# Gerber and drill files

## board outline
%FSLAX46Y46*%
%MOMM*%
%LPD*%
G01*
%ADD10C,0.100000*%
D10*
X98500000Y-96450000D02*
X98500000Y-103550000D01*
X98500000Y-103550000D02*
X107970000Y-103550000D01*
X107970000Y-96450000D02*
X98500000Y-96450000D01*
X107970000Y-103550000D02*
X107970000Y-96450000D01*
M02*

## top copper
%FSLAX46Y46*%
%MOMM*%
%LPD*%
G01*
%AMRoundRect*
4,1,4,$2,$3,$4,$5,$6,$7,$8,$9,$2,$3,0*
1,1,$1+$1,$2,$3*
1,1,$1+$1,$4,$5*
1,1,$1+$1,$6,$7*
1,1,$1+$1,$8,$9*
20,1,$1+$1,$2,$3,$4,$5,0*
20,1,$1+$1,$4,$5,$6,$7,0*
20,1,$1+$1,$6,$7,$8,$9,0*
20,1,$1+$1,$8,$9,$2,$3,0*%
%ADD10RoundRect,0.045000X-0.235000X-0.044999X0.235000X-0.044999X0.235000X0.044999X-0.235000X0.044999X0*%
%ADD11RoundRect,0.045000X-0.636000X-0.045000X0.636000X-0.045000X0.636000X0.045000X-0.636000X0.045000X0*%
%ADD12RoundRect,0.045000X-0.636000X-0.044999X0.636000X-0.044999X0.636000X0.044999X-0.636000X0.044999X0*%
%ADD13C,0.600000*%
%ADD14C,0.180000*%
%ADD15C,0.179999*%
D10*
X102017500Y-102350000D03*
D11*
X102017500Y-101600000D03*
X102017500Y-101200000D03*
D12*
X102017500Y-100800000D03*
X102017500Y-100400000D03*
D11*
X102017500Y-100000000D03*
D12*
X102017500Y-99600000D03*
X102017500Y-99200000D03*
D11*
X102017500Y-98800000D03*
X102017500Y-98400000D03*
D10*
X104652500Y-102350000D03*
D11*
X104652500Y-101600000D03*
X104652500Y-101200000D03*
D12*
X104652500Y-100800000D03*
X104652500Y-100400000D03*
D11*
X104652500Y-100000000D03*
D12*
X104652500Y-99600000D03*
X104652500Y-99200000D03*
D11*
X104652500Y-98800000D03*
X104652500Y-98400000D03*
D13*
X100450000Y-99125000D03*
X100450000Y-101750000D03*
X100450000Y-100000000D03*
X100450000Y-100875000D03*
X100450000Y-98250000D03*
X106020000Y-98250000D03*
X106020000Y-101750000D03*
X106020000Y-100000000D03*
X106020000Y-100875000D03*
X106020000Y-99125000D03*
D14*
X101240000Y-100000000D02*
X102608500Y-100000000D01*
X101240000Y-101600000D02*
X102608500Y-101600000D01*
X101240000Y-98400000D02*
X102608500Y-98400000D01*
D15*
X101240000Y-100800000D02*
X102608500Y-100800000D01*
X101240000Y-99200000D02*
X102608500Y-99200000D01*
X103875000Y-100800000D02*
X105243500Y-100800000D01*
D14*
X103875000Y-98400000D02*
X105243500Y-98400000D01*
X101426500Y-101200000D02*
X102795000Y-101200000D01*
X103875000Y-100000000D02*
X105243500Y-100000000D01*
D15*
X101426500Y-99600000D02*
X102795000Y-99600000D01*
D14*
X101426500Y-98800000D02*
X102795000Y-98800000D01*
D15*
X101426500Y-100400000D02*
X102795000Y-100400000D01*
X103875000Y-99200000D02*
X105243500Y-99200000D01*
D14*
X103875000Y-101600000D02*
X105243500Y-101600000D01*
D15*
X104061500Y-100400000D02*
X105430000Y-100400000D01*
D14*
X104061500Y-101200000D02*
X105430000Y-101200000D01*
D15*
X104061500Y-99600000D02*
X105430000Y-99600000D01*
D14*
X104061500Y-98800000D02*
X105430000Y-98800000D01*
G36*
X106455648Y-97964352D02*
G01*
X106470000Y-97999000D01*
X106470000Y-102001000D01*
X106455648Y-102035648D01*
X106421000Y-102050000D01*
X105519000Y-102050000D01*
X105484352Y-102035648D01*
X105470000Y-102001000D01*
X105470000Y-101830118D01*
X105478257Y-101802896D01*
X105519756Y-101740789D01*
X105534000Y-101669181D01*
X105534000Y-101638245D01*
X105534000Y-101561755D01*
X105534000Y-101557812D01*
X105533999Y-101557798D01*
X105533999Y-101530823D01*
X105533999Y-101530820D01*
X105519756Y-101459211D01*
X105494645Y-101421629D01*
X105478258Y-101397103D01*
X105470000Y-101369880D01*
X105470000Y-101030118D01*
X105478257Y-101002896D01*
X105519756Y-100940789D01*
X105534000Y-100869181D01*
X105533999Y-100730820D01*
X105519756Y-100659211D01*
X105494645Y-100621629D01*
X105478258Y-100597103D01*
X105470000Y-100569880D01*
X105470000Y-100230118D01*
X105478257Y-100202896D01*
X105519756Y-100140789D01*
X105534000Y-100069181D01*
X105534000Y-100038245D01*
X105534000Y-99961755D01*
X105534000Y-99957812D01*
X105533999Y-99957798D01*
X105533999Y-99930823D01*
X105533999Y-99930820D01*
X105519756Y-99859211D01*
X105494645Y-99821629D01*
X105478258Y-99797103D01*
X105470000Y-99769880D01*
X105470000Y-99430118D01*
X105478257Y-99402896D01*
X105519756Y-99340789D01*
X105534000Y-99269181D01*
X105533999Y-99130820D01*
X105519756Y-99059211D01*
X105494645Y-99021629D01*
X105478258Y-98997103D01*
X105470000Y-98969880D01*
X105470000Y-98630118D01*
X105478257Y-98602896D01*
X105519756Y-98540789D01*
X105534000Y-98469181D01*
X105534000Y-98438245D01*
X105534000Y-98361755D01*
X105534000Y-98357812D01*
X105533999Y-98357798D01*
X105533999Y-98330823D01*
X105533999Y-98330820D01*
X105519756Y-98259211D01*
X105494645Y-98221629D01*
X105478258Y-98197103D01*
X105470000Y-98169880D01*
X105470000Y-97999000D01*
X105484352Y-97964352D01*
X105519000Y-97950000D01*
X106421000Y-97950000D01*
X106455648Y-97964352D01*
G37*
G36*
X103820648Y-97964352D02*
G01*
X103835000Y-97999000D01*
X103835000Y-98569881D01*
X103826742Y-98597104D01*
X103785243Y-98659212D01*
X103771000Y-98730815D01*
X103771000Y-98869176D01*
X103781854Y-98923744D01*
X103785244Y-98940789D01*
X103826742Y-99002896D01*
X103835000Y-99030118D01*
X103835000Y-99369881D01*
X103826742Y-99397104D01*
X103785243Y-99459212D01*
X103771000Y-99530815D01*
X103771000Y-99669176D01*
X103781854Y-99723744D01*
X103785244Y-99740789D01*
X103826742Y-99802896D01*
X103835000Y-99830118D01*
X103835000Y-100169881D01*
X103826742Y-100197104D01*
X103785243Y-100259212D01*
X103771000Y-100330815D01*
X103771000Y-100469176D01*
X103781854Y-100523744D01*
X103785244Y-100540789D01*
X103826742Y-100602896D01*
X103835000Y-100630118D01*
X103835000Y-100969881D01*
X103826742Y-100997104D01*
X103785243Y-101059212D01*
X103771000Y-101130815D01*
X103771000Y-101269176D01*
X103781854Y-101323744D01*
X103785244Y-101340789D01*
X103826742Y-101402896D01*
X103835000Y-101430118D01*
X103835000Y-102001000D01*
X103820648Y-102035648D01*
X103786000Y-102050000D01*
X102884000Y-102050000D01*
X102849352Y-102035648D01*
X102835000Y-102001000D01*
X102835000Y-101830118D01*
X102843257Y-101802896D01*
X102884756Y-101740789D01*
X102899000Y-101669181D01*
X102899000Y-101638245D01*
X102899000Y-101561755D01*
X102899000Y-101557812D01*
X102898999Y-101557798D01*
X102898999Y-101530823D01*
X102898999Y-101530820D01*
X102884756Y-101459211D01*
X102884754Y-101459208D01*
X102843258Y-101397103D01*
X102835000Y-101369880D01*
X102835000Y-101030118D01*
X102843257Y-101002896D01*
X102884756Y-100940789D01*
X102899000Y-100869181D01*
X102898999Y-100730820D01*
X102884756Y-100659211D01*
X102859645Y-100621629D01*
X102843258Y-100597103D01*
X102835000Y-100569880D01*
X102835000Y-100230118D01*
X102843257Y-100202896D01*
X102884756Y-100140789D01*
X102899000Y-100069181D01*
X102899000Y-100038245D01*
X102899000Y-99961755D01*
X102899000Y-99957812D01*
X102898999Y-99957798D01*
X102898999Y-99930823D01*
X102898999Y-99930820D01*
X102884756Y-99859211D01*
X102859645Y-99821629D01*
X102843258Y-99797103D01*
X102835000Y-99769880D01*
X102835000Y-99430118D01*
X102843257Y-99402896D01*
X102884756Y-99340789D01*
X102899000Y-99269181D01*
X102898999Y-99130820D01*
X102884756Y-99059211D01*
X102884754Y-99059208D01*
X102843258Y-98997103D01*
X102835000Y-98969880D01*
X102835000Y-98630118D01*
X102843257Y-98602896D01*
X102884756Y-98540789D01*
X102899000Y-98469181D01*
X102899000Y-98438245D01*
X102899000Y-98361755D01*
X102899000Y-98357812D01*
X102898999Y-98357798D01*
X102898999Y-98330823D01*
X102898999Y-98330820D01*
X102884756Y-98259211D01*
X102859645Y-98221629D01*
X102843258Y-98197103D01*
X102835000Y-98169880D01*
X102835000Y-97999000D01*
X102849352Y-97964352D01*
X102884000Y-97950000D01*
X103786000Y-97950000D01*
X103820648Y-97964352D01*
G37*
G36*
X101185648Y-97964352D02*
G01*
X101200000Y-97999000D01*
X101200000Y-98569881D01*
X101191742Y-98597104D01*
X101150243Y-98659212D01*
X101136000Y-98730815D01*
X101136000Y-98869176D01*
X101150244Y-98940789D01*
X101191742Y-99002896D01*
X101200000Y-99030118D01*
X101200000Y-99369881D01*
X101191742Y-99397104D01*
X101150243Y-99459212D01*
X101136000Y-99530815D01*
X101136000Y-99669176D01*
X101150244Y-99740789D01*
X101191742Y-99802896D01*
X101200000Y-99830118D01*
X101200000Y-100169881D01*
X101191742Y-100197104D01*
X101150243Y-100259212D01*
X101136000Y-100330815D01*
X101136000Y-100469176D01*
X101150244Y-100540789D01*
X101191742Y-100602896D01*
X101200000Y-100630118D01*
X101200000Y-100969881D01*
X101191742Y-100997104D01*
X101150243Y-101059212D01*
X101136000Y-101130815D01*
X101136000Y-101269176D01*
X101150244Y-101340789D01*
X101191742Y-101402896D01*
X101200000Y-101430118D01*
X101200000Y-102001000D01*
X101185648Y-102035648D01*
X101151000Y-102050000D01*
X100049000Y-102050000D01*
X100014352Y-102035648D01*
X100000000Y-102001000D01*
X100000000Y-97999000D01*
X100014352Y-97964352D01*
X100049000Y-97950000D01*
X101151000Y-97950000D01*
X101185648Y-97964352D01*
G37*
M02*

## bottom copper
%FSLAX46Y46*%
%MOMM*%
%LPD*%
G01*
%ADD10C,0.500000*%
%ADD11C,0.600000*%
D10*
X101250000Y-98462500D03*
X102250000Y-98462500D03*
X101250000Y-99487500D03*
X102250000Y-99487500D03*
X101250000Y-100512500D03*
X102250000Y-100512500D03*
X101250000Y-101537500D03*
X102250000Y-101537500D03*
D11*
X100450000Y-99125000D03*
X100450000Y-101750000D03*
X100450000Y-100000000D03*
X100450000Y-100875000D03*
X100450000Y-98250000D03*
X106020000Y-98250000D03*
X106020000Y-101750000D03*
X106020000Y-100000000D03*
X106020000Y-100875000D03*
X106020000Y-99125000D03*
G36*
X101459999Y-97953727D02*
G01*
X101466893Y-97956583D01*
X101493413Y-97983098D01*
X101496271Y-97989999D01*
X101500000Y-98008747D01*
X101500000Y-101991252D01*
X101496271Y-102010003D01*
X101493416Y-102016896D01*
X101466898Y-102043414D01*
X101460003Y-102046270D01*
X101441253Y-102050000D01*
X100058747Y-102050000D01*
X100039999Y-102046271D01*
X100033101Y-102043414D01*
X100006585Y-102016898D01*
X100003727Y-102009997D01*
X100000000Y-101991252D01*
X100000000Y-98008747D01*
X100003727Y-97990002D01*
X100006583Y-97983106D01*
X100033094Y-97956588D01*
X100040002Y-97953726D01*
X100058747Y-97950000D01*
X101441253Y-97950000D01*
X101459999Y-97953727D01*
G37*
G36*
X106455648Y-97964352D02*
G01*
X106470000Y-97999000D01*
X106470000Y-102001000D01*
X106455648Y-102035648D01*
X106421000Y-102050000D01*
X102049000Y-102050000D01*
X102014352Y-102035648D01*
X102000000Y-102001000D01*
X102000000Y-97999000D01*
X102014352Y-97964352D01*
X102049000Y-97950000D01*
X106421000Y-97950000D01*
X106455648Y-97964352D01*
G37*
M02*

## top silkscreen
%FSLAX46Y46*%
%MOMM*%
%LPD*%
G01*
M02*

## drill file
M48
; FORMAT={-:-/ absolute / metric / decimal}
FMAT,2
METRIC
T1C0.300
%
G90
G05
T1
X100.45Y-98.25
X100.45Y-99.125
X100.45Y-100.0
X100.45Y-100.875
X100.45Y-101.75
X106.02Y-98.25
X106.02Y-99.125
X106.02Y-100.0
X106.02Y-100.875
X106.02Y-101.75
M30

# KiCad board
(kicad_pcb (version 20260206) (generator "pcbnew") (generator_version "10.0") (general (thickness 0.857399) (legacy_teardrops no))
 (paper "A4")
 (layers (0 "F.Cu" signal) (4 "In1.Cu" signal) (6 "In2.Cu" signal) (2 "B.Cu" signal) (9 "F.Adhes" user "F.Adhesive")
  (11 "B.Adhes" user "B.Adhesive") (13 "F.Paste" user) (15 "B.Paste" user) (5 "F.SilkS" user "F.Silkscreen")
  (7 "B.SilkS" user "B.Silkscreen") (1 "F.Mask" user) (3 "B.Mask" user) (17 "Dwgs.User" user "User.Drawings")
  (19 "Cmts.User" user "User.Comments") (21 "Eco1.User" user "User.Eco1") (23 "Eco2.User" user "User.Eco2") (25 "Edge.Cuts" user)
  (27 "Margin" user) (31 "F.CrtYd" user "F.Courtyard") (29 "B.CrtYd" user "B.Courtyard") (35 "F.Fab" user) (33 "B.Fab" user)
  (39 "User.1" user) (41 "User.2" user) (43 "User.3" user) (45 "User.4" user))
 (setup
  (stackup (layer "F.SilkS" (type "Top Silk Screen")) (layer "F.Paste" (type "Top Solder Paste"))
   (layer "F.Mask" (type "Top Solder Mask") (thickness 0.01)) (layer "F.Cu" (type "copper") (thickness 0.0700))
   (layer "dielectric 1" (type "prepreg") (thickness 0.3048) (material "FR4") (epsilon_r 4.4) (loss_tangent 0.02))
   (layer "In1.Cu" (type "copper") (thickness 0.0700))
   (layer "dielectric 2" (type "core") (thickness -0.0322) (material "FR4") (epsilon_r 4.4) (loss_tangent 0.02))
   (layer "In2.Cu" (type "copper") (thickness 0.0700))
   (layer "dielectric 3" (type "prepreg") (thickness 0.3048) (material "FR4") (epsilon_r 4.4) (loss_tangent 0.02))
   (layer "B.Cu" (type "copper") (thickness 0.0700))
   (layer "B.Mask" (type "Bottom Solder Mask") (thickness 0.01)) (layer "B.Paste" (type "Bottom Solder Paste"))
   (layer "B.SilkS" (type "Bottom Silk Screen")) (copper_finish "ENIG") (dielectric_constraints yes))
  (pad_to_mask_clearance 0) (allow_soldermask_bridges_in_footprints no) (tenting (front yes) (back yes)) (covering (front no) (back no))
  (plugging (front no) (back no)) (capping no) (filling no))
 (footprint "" (layer "F.Cu") (at 0 0)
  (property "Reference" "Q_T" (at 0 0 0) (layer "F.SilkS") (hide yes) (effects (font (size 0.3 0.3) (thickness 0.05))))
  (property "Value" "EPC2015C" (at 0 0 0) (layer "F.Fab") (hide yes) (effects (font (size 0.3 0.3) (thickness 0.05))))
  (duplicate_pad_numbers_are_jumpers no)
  (pad "1" smd roundrect (at 102.0175 102.35) (size 0.56 0.179999) (layers "F.Cu" "F.Mask" "F.Paste") (roundrect_rratio 0.25) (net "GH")
   (thermal_bridge_angle 45))
  (pad "3" smd roundrect (at 102.0175 101.6) (size 1.362 0.18) (layers "F.Cu" "F.Mask" "F.Paste") (roundrect_rratio 0.25) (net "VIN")
   (thermal_bridge_angle 45))
  (pad "4" smd roundrect (at 102.0175 101.2) (size 1.362 0.18) (layers "F.Cu" "F.Mask" "F.Paste") (roundrect_rratio 0.25) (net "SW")
   (thermal_bridge_angle 45))
  (pad "5" smd roundrect (at 102.0175 100.8) (size 1.362 0.179999) (layers "F.Cu" "F.Mask" "F.Paste") (roundrect_rratio 0.25) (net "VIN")
   (thermal_bridge_angle 45))
  (pad "6" smd roundrect (at 102.0175 100.4) (size 1.362 0.179999) (layers "F.Cu" "F.Mask" "F.Paste") (roundrect_rratio 0.25) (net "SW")
   (thermal_bridge_angle 45))
  (pad "7" smd roundrect (at 102.0175 100) (size 1.362 0.18) (layers "F.Cu" "F.Mask" "F.Paste") (roundrect_rratio 0.25) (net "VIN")
   (thermal_bridge_angle 45))
  (pad "8" smd roundrect (at 102.0175 99.6) (size 1.362 0.179999) (layers "F.Cu" "F.Mask" "F.Paste") (roundrect_rratio 0.25) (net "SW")
   (thermal_bridge_angle 45))
  (pad "9" smd roundrect (at 102.0175 99.2) (size 1.362 0.179999) (layers "F.Cu" "F.Mask" "F.Paste") (roundrect_rratio 0.25) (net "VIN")
   (thermal_bridge_angle 45))
  (pad "10" smd roundrect (at 102.0175 98.8) (size 1.362 0.18) (layers "F.Cu" "F.Mask" "F.Paste") (roundrect_rratio 0.25) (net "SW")
   (thermal_bridge_angle 45))
  (pad "11" smd roundrect (at 102.0175 98.4) (size 1.362 0.18) (layers "F.Cu" "F.Mask" "F.Paste") (roundrect_rratio 0.25) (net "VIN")
   (thermal_bridge_angle 45)))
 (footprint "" (layer "F.Cu") (at 0 0)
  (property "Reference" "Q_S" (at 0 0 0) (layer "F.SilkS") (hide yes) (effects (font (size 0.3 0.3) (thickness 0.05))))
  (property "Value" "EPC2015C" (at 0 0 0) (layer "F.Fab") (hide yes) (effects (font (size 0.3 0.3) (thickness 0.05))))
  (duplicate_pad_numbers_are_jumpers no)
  (pad "1" smd roundrect (at 104.6525 102.35) (size 0.56 0.179999) (layers "F.Cu" "F.Mask" "F.Paste") (roundrect_rratio 0.25) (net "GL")
   (thermal_bridge_angle 45))
  (pad "3" smd roundrect (at 104.6525 101.6) (size 1.362 0.18) (layers "F.Cu" "F.Mask" "F.Paste") (roundrect_rratio 0.25) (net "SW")
   (thermal_bridge_angle 45))
  (pad "4" smd roundrect (at 104.6525 101.2) (size 1.362 0.18) (layers "F.Cu" "F.Mask" "F.Paste") (roundrect_rratio 0.25) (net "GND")
   (thermal_bridge_angle 45))
  (pad "5" smd roundrect (at 104.6525 100.8) (size 1.362 0.179999) (layers "F.Cu" "F.Mask" "F.Paste") (roundrect_rratio 0.25) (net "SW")
   (thermal_bridge_angle 45))
  (pad "6" smd roundrect (at 104.6525 100.4) (size 1.362 0.179999) (layers "F.Cu" "F.Mask" "F.Paste") (roundrect_rratio 0.25) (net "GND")
   (thermal_bridge_angle 45))
  (pad "7" smd roundrect (at 104.6525 100) (size 1.362 0.18) (layers "F.Cu" "F.Mask" "F.Paste") (roundrect_rratio 0.25) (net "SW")
   (thermal_bridge_angle 45))
  (pad "8" smd roundrect (at 104.6525 99.6) (size 1.362 0.179999) (layers "F.Cu" "F.Mask" "F.Paste") (roundrect_rratio 0.25) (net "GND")
   (thermal_bridge_angle 45))
  (pad "9" smd roundrect (at 104.6525 99.2) (size 1.362 0.179999) (layers "F.Cu" "F.Mask" "F.Paste") (roundrect_rratio 0.25) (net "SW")
   (thermal_bridge_angle 45))
  (pad "10" smd roundrect (at 104.6525 98.8) (size 1.362 0.18) (layers "F.Cu" "F.Mask" "F.Paste") (roundrect_rratio 0.25) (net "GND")
   (thermal_bridge_angle 45))
  (pad "11" smd roundrect (at 104.6525 98.4) (size 1.362 0.18) (layers "F.Cu" "F.Mask" "F.Paste") (roundrect_rratio 0.25) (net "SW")
   (thermal_bridge_angle 45)))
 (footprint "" (layer "B.Cu") (at 101.75 98.4625)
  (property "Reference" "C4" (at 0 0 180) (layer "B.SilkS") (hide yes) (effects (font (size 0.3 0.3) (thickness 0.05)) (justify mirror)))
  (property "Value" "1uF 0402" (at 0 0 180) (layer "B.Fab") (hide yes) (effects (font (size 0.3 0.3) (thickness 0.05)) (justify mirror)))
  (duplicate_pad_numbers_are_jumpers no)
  (pad "1" smd circle (at -0.5 0) (size 0.5 0.5) (layers "B.Cu" "B.Mask" "B.Paste") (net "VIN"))
  (pad "2" smd circle (at 0.5 0) (size 0.5 0.5) (layers "B.Cu" "B.Mask" "B.Paste") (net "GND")))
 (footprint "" (layer "B.Cu") (at 101.75 99.4875)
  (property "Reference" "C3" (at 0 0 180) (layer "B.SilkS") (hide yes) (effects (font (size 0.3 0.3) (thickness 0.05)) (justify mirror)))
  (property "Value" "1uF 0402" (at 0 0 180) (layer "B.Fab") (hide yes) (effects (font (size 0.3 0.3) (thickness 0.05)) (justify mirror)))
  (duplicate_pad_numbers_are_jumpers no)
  (pad "1" smd circle (at -0.5 0) (size 0.5 0.5) (layers "B.Cu" "B.Mask" "B.Paste") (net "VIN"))
  (pad "2" smd circle (at 0.5 0) (size 0.5 0.5) (layers "B.Cu" "B.Mask" "B.Paste") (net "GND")))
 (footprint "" (layer "B.Cu") (at 101.75 100.5125)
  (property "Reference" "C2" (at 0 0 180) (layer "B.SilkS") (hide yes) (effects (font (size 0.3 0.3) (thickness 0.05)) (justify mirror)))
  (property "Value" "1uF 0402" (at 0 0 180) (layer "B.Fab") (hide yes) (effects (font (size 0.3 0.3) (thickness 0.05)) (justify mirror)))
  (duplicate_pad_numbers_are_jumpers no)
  (pad "1" smd circle (at -0.5 0) (size 0.5 0.5) (layers "B.Cu" "B.Mask" "B.Paste") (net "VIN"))
  (pad "2" smd circle (at 0.5 0) (size 0.5 0.5) (layers "B.Cu" "B.Mask" "B.Paste") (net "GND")))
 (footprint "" (layer "B.Cu") (at 101.75 101.5375)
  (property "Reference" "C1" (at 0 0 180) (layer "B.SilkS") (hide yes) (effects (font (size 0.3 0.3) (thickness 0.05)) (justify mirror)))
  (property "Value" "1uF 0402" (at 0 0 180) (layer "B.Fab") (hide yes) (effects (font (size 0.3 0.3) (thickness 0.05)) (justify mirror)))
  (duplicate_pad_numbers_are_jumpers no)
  (pad "1" smd circle (at -0.5 0) (size 0.5 0.5) (layers "B.Cu" "B.Mask" "B.Paste") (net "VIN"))
  (pad "2" smd circle (at 0.5 0) (size 0.5 0.5) (layers "B.Cu" "B.Mask" "B.Paste") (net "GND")))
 (gr_line (start 98.5 96.45) (end 98.5 103.55) (stroke (width 0.1) (type default)) (layer "Edge.Cuts"))
 (gr_line (start 98.5 103.55) (end 107.97 103.55) (stroke (width 0.1) (type default)) (layer "Edge.Cuts"))
 (gr_line (start 107.97 96.45) (end 98.5 96.45) (stroke (width 0.1) (type default)) (layer "Edge.Cuts"))
 (gr_line (start 107.97 103.55) (end 107.97 96.45) (stroke (width 0.1) (type default)) (layer "Edge.Cuts"))
 (segment (start 101.24 100) (end 102.6085 100) (width 0.18) (layer "F.Cu") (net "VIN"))
 (segment (start 101.24 101.6) (end 102.6085 101.6) (width 0.18) (layer "F.Cu") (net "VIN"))
 (segment (start 101.24 98.4) (end 102.6085 98.4) (width 0.18) (layer "F.Cu") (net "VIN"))
 (segment (start 101.24 100.8) (end 102.6085 100.8) (width 0.179999) (layer "F.Cu") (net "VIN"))
 (segment (start 101.24 99.2) (end 102.6085 99.2) (width 0.179999) (layer "F.Cu") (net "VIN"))
 (via (at 100.45 99.125) (size 0.6) (drill 0.3) (layers "F.Cu" "B.Cu") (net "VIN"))
 (via (at 100.45 101.75) (size 0.6) (drill 0.3) (layers "F.Cu" "B.Cu") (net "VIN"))
 (via (at 100.45 100) (size 0.6) (drill 0.3) (layers "F.Cu" "B.Cu") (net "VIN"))
 (via (at 100.45 100.875) (size 0.6) (drill 0.3) (layers "F.Cu" "B.Cu") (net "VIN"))
 (via (at 100.45 98.25) (size 0.6) (drill 0.3) (layers "F.Cu" "B.Cu") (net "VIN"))
 (segment (start 103.875 100.8) (end 105.2435 100.8) (width 0.179999) (layer "F.Cu") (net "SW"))
 (segment (start 103.875 98.4) (end 105.2435 98.4) (width 0.18) (layer "F.Cu") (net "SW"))
 (segment (start 101.4265 101.2) (end 102.795 101.2) (width 0.18) (layer "F.Cu") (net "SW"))
 (segment (start 103.875 100) (end 105.2435 100) (width 0.18) (layer "F.Cu") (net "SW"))
 (segment (start 101.4265 99.6) (end 102.795 99.6) (width 0.179999) (layer "F.Cu") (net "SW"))
 (segment (start 101.4265 98.8) (end 102.795 98.8) (width 0.18) (layer "F.Cu") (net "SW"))
 (segment (start 101.4265 100.4) (end 102.795 100.4) (width 0.179999) (layer "F.Cu") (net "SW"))
 (segment (start 103.875 99.2) (end 105.2435 99.2) (width 0.179999) (layer "F.Cu") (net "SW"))
 (segment (start 103.875 101.6) (end 105.2435 101.6) (width 0.18) (layer "F.Cu") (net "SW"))
 (segment (start 104.0615 100.4) (end 105.43 100.4) (width 0.179999) (layer "F.Cu") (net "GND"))
 (segment (start 104.0615 101.2) (end 105.43 101.2) (width 0.18) (layer "F.Cu") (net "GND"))
 (segment (start 104.0615 99.6) (end 105.43 99.6) (width 0.179999) (layer "F.Cu") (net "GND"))
 (segment (start 104.0615 98.8) (end 105.43 98.8) (width 0.18) (layer "F.Cu") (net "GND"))
 (via (at 106.02 98.25) (size 0.6) (drill 0.3) (layers "F.Cu" "B.Cu") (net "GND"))
 (via (at 106.02 101.75) (size 0.6) (drill 0.3) (layers "F.Cu" "B.Cu") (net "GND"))
 (via (at 106.02 100) (size 0.6) (drill 0.3) (layers "F.Cu" "B.Cu") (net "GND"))
 (via (at 106.02 100.875) (size 0.6) (drill 0.3) (layers "F.Cu" "B.Cu") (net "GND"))
 (via (at 106.02 99.125) (size 0.6) (drill 0.3) (layers "F.Cu" "B.Cu") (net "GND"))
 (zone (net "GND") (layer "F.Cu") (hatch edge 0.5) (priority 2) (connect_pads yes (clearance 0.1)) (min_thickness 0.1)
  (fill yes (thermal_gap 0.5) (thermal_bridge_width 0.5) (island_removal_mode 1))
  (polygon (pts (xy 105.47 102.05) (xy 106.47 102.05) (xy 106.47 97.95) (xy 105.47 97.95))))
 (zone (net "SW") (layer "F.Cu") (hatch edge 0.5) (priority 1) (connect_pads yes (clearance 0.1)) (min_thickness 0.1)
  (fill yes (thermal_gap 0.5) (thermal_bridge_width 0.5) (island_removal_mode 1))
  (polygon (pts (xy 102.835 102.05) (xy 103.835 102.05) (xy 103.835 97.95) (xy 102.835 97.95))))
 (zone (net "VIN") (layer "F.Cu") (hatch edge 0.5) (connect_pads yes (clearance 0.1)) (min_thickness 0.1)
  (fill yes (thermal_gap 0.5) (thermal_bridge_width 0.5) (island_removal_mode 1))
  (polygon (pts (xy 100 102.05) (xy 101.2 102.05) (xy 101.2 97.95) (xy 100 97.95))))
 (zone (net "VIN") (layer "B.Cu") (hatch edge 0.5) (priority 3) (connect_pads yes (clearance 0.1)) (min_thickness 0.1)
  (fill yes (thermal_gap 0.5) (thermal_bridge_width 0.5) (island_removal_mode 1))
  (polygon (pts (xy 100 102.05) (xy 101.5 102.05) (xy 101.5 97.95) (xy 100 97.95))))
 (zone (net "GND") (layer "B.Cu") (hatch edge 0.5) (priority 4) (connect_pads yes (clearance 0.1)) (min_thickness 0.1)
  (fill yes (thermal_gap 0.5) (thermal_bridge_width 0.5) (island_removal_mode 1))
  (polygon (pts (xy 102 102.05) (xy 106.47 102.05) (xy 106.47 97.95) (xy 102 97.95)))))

